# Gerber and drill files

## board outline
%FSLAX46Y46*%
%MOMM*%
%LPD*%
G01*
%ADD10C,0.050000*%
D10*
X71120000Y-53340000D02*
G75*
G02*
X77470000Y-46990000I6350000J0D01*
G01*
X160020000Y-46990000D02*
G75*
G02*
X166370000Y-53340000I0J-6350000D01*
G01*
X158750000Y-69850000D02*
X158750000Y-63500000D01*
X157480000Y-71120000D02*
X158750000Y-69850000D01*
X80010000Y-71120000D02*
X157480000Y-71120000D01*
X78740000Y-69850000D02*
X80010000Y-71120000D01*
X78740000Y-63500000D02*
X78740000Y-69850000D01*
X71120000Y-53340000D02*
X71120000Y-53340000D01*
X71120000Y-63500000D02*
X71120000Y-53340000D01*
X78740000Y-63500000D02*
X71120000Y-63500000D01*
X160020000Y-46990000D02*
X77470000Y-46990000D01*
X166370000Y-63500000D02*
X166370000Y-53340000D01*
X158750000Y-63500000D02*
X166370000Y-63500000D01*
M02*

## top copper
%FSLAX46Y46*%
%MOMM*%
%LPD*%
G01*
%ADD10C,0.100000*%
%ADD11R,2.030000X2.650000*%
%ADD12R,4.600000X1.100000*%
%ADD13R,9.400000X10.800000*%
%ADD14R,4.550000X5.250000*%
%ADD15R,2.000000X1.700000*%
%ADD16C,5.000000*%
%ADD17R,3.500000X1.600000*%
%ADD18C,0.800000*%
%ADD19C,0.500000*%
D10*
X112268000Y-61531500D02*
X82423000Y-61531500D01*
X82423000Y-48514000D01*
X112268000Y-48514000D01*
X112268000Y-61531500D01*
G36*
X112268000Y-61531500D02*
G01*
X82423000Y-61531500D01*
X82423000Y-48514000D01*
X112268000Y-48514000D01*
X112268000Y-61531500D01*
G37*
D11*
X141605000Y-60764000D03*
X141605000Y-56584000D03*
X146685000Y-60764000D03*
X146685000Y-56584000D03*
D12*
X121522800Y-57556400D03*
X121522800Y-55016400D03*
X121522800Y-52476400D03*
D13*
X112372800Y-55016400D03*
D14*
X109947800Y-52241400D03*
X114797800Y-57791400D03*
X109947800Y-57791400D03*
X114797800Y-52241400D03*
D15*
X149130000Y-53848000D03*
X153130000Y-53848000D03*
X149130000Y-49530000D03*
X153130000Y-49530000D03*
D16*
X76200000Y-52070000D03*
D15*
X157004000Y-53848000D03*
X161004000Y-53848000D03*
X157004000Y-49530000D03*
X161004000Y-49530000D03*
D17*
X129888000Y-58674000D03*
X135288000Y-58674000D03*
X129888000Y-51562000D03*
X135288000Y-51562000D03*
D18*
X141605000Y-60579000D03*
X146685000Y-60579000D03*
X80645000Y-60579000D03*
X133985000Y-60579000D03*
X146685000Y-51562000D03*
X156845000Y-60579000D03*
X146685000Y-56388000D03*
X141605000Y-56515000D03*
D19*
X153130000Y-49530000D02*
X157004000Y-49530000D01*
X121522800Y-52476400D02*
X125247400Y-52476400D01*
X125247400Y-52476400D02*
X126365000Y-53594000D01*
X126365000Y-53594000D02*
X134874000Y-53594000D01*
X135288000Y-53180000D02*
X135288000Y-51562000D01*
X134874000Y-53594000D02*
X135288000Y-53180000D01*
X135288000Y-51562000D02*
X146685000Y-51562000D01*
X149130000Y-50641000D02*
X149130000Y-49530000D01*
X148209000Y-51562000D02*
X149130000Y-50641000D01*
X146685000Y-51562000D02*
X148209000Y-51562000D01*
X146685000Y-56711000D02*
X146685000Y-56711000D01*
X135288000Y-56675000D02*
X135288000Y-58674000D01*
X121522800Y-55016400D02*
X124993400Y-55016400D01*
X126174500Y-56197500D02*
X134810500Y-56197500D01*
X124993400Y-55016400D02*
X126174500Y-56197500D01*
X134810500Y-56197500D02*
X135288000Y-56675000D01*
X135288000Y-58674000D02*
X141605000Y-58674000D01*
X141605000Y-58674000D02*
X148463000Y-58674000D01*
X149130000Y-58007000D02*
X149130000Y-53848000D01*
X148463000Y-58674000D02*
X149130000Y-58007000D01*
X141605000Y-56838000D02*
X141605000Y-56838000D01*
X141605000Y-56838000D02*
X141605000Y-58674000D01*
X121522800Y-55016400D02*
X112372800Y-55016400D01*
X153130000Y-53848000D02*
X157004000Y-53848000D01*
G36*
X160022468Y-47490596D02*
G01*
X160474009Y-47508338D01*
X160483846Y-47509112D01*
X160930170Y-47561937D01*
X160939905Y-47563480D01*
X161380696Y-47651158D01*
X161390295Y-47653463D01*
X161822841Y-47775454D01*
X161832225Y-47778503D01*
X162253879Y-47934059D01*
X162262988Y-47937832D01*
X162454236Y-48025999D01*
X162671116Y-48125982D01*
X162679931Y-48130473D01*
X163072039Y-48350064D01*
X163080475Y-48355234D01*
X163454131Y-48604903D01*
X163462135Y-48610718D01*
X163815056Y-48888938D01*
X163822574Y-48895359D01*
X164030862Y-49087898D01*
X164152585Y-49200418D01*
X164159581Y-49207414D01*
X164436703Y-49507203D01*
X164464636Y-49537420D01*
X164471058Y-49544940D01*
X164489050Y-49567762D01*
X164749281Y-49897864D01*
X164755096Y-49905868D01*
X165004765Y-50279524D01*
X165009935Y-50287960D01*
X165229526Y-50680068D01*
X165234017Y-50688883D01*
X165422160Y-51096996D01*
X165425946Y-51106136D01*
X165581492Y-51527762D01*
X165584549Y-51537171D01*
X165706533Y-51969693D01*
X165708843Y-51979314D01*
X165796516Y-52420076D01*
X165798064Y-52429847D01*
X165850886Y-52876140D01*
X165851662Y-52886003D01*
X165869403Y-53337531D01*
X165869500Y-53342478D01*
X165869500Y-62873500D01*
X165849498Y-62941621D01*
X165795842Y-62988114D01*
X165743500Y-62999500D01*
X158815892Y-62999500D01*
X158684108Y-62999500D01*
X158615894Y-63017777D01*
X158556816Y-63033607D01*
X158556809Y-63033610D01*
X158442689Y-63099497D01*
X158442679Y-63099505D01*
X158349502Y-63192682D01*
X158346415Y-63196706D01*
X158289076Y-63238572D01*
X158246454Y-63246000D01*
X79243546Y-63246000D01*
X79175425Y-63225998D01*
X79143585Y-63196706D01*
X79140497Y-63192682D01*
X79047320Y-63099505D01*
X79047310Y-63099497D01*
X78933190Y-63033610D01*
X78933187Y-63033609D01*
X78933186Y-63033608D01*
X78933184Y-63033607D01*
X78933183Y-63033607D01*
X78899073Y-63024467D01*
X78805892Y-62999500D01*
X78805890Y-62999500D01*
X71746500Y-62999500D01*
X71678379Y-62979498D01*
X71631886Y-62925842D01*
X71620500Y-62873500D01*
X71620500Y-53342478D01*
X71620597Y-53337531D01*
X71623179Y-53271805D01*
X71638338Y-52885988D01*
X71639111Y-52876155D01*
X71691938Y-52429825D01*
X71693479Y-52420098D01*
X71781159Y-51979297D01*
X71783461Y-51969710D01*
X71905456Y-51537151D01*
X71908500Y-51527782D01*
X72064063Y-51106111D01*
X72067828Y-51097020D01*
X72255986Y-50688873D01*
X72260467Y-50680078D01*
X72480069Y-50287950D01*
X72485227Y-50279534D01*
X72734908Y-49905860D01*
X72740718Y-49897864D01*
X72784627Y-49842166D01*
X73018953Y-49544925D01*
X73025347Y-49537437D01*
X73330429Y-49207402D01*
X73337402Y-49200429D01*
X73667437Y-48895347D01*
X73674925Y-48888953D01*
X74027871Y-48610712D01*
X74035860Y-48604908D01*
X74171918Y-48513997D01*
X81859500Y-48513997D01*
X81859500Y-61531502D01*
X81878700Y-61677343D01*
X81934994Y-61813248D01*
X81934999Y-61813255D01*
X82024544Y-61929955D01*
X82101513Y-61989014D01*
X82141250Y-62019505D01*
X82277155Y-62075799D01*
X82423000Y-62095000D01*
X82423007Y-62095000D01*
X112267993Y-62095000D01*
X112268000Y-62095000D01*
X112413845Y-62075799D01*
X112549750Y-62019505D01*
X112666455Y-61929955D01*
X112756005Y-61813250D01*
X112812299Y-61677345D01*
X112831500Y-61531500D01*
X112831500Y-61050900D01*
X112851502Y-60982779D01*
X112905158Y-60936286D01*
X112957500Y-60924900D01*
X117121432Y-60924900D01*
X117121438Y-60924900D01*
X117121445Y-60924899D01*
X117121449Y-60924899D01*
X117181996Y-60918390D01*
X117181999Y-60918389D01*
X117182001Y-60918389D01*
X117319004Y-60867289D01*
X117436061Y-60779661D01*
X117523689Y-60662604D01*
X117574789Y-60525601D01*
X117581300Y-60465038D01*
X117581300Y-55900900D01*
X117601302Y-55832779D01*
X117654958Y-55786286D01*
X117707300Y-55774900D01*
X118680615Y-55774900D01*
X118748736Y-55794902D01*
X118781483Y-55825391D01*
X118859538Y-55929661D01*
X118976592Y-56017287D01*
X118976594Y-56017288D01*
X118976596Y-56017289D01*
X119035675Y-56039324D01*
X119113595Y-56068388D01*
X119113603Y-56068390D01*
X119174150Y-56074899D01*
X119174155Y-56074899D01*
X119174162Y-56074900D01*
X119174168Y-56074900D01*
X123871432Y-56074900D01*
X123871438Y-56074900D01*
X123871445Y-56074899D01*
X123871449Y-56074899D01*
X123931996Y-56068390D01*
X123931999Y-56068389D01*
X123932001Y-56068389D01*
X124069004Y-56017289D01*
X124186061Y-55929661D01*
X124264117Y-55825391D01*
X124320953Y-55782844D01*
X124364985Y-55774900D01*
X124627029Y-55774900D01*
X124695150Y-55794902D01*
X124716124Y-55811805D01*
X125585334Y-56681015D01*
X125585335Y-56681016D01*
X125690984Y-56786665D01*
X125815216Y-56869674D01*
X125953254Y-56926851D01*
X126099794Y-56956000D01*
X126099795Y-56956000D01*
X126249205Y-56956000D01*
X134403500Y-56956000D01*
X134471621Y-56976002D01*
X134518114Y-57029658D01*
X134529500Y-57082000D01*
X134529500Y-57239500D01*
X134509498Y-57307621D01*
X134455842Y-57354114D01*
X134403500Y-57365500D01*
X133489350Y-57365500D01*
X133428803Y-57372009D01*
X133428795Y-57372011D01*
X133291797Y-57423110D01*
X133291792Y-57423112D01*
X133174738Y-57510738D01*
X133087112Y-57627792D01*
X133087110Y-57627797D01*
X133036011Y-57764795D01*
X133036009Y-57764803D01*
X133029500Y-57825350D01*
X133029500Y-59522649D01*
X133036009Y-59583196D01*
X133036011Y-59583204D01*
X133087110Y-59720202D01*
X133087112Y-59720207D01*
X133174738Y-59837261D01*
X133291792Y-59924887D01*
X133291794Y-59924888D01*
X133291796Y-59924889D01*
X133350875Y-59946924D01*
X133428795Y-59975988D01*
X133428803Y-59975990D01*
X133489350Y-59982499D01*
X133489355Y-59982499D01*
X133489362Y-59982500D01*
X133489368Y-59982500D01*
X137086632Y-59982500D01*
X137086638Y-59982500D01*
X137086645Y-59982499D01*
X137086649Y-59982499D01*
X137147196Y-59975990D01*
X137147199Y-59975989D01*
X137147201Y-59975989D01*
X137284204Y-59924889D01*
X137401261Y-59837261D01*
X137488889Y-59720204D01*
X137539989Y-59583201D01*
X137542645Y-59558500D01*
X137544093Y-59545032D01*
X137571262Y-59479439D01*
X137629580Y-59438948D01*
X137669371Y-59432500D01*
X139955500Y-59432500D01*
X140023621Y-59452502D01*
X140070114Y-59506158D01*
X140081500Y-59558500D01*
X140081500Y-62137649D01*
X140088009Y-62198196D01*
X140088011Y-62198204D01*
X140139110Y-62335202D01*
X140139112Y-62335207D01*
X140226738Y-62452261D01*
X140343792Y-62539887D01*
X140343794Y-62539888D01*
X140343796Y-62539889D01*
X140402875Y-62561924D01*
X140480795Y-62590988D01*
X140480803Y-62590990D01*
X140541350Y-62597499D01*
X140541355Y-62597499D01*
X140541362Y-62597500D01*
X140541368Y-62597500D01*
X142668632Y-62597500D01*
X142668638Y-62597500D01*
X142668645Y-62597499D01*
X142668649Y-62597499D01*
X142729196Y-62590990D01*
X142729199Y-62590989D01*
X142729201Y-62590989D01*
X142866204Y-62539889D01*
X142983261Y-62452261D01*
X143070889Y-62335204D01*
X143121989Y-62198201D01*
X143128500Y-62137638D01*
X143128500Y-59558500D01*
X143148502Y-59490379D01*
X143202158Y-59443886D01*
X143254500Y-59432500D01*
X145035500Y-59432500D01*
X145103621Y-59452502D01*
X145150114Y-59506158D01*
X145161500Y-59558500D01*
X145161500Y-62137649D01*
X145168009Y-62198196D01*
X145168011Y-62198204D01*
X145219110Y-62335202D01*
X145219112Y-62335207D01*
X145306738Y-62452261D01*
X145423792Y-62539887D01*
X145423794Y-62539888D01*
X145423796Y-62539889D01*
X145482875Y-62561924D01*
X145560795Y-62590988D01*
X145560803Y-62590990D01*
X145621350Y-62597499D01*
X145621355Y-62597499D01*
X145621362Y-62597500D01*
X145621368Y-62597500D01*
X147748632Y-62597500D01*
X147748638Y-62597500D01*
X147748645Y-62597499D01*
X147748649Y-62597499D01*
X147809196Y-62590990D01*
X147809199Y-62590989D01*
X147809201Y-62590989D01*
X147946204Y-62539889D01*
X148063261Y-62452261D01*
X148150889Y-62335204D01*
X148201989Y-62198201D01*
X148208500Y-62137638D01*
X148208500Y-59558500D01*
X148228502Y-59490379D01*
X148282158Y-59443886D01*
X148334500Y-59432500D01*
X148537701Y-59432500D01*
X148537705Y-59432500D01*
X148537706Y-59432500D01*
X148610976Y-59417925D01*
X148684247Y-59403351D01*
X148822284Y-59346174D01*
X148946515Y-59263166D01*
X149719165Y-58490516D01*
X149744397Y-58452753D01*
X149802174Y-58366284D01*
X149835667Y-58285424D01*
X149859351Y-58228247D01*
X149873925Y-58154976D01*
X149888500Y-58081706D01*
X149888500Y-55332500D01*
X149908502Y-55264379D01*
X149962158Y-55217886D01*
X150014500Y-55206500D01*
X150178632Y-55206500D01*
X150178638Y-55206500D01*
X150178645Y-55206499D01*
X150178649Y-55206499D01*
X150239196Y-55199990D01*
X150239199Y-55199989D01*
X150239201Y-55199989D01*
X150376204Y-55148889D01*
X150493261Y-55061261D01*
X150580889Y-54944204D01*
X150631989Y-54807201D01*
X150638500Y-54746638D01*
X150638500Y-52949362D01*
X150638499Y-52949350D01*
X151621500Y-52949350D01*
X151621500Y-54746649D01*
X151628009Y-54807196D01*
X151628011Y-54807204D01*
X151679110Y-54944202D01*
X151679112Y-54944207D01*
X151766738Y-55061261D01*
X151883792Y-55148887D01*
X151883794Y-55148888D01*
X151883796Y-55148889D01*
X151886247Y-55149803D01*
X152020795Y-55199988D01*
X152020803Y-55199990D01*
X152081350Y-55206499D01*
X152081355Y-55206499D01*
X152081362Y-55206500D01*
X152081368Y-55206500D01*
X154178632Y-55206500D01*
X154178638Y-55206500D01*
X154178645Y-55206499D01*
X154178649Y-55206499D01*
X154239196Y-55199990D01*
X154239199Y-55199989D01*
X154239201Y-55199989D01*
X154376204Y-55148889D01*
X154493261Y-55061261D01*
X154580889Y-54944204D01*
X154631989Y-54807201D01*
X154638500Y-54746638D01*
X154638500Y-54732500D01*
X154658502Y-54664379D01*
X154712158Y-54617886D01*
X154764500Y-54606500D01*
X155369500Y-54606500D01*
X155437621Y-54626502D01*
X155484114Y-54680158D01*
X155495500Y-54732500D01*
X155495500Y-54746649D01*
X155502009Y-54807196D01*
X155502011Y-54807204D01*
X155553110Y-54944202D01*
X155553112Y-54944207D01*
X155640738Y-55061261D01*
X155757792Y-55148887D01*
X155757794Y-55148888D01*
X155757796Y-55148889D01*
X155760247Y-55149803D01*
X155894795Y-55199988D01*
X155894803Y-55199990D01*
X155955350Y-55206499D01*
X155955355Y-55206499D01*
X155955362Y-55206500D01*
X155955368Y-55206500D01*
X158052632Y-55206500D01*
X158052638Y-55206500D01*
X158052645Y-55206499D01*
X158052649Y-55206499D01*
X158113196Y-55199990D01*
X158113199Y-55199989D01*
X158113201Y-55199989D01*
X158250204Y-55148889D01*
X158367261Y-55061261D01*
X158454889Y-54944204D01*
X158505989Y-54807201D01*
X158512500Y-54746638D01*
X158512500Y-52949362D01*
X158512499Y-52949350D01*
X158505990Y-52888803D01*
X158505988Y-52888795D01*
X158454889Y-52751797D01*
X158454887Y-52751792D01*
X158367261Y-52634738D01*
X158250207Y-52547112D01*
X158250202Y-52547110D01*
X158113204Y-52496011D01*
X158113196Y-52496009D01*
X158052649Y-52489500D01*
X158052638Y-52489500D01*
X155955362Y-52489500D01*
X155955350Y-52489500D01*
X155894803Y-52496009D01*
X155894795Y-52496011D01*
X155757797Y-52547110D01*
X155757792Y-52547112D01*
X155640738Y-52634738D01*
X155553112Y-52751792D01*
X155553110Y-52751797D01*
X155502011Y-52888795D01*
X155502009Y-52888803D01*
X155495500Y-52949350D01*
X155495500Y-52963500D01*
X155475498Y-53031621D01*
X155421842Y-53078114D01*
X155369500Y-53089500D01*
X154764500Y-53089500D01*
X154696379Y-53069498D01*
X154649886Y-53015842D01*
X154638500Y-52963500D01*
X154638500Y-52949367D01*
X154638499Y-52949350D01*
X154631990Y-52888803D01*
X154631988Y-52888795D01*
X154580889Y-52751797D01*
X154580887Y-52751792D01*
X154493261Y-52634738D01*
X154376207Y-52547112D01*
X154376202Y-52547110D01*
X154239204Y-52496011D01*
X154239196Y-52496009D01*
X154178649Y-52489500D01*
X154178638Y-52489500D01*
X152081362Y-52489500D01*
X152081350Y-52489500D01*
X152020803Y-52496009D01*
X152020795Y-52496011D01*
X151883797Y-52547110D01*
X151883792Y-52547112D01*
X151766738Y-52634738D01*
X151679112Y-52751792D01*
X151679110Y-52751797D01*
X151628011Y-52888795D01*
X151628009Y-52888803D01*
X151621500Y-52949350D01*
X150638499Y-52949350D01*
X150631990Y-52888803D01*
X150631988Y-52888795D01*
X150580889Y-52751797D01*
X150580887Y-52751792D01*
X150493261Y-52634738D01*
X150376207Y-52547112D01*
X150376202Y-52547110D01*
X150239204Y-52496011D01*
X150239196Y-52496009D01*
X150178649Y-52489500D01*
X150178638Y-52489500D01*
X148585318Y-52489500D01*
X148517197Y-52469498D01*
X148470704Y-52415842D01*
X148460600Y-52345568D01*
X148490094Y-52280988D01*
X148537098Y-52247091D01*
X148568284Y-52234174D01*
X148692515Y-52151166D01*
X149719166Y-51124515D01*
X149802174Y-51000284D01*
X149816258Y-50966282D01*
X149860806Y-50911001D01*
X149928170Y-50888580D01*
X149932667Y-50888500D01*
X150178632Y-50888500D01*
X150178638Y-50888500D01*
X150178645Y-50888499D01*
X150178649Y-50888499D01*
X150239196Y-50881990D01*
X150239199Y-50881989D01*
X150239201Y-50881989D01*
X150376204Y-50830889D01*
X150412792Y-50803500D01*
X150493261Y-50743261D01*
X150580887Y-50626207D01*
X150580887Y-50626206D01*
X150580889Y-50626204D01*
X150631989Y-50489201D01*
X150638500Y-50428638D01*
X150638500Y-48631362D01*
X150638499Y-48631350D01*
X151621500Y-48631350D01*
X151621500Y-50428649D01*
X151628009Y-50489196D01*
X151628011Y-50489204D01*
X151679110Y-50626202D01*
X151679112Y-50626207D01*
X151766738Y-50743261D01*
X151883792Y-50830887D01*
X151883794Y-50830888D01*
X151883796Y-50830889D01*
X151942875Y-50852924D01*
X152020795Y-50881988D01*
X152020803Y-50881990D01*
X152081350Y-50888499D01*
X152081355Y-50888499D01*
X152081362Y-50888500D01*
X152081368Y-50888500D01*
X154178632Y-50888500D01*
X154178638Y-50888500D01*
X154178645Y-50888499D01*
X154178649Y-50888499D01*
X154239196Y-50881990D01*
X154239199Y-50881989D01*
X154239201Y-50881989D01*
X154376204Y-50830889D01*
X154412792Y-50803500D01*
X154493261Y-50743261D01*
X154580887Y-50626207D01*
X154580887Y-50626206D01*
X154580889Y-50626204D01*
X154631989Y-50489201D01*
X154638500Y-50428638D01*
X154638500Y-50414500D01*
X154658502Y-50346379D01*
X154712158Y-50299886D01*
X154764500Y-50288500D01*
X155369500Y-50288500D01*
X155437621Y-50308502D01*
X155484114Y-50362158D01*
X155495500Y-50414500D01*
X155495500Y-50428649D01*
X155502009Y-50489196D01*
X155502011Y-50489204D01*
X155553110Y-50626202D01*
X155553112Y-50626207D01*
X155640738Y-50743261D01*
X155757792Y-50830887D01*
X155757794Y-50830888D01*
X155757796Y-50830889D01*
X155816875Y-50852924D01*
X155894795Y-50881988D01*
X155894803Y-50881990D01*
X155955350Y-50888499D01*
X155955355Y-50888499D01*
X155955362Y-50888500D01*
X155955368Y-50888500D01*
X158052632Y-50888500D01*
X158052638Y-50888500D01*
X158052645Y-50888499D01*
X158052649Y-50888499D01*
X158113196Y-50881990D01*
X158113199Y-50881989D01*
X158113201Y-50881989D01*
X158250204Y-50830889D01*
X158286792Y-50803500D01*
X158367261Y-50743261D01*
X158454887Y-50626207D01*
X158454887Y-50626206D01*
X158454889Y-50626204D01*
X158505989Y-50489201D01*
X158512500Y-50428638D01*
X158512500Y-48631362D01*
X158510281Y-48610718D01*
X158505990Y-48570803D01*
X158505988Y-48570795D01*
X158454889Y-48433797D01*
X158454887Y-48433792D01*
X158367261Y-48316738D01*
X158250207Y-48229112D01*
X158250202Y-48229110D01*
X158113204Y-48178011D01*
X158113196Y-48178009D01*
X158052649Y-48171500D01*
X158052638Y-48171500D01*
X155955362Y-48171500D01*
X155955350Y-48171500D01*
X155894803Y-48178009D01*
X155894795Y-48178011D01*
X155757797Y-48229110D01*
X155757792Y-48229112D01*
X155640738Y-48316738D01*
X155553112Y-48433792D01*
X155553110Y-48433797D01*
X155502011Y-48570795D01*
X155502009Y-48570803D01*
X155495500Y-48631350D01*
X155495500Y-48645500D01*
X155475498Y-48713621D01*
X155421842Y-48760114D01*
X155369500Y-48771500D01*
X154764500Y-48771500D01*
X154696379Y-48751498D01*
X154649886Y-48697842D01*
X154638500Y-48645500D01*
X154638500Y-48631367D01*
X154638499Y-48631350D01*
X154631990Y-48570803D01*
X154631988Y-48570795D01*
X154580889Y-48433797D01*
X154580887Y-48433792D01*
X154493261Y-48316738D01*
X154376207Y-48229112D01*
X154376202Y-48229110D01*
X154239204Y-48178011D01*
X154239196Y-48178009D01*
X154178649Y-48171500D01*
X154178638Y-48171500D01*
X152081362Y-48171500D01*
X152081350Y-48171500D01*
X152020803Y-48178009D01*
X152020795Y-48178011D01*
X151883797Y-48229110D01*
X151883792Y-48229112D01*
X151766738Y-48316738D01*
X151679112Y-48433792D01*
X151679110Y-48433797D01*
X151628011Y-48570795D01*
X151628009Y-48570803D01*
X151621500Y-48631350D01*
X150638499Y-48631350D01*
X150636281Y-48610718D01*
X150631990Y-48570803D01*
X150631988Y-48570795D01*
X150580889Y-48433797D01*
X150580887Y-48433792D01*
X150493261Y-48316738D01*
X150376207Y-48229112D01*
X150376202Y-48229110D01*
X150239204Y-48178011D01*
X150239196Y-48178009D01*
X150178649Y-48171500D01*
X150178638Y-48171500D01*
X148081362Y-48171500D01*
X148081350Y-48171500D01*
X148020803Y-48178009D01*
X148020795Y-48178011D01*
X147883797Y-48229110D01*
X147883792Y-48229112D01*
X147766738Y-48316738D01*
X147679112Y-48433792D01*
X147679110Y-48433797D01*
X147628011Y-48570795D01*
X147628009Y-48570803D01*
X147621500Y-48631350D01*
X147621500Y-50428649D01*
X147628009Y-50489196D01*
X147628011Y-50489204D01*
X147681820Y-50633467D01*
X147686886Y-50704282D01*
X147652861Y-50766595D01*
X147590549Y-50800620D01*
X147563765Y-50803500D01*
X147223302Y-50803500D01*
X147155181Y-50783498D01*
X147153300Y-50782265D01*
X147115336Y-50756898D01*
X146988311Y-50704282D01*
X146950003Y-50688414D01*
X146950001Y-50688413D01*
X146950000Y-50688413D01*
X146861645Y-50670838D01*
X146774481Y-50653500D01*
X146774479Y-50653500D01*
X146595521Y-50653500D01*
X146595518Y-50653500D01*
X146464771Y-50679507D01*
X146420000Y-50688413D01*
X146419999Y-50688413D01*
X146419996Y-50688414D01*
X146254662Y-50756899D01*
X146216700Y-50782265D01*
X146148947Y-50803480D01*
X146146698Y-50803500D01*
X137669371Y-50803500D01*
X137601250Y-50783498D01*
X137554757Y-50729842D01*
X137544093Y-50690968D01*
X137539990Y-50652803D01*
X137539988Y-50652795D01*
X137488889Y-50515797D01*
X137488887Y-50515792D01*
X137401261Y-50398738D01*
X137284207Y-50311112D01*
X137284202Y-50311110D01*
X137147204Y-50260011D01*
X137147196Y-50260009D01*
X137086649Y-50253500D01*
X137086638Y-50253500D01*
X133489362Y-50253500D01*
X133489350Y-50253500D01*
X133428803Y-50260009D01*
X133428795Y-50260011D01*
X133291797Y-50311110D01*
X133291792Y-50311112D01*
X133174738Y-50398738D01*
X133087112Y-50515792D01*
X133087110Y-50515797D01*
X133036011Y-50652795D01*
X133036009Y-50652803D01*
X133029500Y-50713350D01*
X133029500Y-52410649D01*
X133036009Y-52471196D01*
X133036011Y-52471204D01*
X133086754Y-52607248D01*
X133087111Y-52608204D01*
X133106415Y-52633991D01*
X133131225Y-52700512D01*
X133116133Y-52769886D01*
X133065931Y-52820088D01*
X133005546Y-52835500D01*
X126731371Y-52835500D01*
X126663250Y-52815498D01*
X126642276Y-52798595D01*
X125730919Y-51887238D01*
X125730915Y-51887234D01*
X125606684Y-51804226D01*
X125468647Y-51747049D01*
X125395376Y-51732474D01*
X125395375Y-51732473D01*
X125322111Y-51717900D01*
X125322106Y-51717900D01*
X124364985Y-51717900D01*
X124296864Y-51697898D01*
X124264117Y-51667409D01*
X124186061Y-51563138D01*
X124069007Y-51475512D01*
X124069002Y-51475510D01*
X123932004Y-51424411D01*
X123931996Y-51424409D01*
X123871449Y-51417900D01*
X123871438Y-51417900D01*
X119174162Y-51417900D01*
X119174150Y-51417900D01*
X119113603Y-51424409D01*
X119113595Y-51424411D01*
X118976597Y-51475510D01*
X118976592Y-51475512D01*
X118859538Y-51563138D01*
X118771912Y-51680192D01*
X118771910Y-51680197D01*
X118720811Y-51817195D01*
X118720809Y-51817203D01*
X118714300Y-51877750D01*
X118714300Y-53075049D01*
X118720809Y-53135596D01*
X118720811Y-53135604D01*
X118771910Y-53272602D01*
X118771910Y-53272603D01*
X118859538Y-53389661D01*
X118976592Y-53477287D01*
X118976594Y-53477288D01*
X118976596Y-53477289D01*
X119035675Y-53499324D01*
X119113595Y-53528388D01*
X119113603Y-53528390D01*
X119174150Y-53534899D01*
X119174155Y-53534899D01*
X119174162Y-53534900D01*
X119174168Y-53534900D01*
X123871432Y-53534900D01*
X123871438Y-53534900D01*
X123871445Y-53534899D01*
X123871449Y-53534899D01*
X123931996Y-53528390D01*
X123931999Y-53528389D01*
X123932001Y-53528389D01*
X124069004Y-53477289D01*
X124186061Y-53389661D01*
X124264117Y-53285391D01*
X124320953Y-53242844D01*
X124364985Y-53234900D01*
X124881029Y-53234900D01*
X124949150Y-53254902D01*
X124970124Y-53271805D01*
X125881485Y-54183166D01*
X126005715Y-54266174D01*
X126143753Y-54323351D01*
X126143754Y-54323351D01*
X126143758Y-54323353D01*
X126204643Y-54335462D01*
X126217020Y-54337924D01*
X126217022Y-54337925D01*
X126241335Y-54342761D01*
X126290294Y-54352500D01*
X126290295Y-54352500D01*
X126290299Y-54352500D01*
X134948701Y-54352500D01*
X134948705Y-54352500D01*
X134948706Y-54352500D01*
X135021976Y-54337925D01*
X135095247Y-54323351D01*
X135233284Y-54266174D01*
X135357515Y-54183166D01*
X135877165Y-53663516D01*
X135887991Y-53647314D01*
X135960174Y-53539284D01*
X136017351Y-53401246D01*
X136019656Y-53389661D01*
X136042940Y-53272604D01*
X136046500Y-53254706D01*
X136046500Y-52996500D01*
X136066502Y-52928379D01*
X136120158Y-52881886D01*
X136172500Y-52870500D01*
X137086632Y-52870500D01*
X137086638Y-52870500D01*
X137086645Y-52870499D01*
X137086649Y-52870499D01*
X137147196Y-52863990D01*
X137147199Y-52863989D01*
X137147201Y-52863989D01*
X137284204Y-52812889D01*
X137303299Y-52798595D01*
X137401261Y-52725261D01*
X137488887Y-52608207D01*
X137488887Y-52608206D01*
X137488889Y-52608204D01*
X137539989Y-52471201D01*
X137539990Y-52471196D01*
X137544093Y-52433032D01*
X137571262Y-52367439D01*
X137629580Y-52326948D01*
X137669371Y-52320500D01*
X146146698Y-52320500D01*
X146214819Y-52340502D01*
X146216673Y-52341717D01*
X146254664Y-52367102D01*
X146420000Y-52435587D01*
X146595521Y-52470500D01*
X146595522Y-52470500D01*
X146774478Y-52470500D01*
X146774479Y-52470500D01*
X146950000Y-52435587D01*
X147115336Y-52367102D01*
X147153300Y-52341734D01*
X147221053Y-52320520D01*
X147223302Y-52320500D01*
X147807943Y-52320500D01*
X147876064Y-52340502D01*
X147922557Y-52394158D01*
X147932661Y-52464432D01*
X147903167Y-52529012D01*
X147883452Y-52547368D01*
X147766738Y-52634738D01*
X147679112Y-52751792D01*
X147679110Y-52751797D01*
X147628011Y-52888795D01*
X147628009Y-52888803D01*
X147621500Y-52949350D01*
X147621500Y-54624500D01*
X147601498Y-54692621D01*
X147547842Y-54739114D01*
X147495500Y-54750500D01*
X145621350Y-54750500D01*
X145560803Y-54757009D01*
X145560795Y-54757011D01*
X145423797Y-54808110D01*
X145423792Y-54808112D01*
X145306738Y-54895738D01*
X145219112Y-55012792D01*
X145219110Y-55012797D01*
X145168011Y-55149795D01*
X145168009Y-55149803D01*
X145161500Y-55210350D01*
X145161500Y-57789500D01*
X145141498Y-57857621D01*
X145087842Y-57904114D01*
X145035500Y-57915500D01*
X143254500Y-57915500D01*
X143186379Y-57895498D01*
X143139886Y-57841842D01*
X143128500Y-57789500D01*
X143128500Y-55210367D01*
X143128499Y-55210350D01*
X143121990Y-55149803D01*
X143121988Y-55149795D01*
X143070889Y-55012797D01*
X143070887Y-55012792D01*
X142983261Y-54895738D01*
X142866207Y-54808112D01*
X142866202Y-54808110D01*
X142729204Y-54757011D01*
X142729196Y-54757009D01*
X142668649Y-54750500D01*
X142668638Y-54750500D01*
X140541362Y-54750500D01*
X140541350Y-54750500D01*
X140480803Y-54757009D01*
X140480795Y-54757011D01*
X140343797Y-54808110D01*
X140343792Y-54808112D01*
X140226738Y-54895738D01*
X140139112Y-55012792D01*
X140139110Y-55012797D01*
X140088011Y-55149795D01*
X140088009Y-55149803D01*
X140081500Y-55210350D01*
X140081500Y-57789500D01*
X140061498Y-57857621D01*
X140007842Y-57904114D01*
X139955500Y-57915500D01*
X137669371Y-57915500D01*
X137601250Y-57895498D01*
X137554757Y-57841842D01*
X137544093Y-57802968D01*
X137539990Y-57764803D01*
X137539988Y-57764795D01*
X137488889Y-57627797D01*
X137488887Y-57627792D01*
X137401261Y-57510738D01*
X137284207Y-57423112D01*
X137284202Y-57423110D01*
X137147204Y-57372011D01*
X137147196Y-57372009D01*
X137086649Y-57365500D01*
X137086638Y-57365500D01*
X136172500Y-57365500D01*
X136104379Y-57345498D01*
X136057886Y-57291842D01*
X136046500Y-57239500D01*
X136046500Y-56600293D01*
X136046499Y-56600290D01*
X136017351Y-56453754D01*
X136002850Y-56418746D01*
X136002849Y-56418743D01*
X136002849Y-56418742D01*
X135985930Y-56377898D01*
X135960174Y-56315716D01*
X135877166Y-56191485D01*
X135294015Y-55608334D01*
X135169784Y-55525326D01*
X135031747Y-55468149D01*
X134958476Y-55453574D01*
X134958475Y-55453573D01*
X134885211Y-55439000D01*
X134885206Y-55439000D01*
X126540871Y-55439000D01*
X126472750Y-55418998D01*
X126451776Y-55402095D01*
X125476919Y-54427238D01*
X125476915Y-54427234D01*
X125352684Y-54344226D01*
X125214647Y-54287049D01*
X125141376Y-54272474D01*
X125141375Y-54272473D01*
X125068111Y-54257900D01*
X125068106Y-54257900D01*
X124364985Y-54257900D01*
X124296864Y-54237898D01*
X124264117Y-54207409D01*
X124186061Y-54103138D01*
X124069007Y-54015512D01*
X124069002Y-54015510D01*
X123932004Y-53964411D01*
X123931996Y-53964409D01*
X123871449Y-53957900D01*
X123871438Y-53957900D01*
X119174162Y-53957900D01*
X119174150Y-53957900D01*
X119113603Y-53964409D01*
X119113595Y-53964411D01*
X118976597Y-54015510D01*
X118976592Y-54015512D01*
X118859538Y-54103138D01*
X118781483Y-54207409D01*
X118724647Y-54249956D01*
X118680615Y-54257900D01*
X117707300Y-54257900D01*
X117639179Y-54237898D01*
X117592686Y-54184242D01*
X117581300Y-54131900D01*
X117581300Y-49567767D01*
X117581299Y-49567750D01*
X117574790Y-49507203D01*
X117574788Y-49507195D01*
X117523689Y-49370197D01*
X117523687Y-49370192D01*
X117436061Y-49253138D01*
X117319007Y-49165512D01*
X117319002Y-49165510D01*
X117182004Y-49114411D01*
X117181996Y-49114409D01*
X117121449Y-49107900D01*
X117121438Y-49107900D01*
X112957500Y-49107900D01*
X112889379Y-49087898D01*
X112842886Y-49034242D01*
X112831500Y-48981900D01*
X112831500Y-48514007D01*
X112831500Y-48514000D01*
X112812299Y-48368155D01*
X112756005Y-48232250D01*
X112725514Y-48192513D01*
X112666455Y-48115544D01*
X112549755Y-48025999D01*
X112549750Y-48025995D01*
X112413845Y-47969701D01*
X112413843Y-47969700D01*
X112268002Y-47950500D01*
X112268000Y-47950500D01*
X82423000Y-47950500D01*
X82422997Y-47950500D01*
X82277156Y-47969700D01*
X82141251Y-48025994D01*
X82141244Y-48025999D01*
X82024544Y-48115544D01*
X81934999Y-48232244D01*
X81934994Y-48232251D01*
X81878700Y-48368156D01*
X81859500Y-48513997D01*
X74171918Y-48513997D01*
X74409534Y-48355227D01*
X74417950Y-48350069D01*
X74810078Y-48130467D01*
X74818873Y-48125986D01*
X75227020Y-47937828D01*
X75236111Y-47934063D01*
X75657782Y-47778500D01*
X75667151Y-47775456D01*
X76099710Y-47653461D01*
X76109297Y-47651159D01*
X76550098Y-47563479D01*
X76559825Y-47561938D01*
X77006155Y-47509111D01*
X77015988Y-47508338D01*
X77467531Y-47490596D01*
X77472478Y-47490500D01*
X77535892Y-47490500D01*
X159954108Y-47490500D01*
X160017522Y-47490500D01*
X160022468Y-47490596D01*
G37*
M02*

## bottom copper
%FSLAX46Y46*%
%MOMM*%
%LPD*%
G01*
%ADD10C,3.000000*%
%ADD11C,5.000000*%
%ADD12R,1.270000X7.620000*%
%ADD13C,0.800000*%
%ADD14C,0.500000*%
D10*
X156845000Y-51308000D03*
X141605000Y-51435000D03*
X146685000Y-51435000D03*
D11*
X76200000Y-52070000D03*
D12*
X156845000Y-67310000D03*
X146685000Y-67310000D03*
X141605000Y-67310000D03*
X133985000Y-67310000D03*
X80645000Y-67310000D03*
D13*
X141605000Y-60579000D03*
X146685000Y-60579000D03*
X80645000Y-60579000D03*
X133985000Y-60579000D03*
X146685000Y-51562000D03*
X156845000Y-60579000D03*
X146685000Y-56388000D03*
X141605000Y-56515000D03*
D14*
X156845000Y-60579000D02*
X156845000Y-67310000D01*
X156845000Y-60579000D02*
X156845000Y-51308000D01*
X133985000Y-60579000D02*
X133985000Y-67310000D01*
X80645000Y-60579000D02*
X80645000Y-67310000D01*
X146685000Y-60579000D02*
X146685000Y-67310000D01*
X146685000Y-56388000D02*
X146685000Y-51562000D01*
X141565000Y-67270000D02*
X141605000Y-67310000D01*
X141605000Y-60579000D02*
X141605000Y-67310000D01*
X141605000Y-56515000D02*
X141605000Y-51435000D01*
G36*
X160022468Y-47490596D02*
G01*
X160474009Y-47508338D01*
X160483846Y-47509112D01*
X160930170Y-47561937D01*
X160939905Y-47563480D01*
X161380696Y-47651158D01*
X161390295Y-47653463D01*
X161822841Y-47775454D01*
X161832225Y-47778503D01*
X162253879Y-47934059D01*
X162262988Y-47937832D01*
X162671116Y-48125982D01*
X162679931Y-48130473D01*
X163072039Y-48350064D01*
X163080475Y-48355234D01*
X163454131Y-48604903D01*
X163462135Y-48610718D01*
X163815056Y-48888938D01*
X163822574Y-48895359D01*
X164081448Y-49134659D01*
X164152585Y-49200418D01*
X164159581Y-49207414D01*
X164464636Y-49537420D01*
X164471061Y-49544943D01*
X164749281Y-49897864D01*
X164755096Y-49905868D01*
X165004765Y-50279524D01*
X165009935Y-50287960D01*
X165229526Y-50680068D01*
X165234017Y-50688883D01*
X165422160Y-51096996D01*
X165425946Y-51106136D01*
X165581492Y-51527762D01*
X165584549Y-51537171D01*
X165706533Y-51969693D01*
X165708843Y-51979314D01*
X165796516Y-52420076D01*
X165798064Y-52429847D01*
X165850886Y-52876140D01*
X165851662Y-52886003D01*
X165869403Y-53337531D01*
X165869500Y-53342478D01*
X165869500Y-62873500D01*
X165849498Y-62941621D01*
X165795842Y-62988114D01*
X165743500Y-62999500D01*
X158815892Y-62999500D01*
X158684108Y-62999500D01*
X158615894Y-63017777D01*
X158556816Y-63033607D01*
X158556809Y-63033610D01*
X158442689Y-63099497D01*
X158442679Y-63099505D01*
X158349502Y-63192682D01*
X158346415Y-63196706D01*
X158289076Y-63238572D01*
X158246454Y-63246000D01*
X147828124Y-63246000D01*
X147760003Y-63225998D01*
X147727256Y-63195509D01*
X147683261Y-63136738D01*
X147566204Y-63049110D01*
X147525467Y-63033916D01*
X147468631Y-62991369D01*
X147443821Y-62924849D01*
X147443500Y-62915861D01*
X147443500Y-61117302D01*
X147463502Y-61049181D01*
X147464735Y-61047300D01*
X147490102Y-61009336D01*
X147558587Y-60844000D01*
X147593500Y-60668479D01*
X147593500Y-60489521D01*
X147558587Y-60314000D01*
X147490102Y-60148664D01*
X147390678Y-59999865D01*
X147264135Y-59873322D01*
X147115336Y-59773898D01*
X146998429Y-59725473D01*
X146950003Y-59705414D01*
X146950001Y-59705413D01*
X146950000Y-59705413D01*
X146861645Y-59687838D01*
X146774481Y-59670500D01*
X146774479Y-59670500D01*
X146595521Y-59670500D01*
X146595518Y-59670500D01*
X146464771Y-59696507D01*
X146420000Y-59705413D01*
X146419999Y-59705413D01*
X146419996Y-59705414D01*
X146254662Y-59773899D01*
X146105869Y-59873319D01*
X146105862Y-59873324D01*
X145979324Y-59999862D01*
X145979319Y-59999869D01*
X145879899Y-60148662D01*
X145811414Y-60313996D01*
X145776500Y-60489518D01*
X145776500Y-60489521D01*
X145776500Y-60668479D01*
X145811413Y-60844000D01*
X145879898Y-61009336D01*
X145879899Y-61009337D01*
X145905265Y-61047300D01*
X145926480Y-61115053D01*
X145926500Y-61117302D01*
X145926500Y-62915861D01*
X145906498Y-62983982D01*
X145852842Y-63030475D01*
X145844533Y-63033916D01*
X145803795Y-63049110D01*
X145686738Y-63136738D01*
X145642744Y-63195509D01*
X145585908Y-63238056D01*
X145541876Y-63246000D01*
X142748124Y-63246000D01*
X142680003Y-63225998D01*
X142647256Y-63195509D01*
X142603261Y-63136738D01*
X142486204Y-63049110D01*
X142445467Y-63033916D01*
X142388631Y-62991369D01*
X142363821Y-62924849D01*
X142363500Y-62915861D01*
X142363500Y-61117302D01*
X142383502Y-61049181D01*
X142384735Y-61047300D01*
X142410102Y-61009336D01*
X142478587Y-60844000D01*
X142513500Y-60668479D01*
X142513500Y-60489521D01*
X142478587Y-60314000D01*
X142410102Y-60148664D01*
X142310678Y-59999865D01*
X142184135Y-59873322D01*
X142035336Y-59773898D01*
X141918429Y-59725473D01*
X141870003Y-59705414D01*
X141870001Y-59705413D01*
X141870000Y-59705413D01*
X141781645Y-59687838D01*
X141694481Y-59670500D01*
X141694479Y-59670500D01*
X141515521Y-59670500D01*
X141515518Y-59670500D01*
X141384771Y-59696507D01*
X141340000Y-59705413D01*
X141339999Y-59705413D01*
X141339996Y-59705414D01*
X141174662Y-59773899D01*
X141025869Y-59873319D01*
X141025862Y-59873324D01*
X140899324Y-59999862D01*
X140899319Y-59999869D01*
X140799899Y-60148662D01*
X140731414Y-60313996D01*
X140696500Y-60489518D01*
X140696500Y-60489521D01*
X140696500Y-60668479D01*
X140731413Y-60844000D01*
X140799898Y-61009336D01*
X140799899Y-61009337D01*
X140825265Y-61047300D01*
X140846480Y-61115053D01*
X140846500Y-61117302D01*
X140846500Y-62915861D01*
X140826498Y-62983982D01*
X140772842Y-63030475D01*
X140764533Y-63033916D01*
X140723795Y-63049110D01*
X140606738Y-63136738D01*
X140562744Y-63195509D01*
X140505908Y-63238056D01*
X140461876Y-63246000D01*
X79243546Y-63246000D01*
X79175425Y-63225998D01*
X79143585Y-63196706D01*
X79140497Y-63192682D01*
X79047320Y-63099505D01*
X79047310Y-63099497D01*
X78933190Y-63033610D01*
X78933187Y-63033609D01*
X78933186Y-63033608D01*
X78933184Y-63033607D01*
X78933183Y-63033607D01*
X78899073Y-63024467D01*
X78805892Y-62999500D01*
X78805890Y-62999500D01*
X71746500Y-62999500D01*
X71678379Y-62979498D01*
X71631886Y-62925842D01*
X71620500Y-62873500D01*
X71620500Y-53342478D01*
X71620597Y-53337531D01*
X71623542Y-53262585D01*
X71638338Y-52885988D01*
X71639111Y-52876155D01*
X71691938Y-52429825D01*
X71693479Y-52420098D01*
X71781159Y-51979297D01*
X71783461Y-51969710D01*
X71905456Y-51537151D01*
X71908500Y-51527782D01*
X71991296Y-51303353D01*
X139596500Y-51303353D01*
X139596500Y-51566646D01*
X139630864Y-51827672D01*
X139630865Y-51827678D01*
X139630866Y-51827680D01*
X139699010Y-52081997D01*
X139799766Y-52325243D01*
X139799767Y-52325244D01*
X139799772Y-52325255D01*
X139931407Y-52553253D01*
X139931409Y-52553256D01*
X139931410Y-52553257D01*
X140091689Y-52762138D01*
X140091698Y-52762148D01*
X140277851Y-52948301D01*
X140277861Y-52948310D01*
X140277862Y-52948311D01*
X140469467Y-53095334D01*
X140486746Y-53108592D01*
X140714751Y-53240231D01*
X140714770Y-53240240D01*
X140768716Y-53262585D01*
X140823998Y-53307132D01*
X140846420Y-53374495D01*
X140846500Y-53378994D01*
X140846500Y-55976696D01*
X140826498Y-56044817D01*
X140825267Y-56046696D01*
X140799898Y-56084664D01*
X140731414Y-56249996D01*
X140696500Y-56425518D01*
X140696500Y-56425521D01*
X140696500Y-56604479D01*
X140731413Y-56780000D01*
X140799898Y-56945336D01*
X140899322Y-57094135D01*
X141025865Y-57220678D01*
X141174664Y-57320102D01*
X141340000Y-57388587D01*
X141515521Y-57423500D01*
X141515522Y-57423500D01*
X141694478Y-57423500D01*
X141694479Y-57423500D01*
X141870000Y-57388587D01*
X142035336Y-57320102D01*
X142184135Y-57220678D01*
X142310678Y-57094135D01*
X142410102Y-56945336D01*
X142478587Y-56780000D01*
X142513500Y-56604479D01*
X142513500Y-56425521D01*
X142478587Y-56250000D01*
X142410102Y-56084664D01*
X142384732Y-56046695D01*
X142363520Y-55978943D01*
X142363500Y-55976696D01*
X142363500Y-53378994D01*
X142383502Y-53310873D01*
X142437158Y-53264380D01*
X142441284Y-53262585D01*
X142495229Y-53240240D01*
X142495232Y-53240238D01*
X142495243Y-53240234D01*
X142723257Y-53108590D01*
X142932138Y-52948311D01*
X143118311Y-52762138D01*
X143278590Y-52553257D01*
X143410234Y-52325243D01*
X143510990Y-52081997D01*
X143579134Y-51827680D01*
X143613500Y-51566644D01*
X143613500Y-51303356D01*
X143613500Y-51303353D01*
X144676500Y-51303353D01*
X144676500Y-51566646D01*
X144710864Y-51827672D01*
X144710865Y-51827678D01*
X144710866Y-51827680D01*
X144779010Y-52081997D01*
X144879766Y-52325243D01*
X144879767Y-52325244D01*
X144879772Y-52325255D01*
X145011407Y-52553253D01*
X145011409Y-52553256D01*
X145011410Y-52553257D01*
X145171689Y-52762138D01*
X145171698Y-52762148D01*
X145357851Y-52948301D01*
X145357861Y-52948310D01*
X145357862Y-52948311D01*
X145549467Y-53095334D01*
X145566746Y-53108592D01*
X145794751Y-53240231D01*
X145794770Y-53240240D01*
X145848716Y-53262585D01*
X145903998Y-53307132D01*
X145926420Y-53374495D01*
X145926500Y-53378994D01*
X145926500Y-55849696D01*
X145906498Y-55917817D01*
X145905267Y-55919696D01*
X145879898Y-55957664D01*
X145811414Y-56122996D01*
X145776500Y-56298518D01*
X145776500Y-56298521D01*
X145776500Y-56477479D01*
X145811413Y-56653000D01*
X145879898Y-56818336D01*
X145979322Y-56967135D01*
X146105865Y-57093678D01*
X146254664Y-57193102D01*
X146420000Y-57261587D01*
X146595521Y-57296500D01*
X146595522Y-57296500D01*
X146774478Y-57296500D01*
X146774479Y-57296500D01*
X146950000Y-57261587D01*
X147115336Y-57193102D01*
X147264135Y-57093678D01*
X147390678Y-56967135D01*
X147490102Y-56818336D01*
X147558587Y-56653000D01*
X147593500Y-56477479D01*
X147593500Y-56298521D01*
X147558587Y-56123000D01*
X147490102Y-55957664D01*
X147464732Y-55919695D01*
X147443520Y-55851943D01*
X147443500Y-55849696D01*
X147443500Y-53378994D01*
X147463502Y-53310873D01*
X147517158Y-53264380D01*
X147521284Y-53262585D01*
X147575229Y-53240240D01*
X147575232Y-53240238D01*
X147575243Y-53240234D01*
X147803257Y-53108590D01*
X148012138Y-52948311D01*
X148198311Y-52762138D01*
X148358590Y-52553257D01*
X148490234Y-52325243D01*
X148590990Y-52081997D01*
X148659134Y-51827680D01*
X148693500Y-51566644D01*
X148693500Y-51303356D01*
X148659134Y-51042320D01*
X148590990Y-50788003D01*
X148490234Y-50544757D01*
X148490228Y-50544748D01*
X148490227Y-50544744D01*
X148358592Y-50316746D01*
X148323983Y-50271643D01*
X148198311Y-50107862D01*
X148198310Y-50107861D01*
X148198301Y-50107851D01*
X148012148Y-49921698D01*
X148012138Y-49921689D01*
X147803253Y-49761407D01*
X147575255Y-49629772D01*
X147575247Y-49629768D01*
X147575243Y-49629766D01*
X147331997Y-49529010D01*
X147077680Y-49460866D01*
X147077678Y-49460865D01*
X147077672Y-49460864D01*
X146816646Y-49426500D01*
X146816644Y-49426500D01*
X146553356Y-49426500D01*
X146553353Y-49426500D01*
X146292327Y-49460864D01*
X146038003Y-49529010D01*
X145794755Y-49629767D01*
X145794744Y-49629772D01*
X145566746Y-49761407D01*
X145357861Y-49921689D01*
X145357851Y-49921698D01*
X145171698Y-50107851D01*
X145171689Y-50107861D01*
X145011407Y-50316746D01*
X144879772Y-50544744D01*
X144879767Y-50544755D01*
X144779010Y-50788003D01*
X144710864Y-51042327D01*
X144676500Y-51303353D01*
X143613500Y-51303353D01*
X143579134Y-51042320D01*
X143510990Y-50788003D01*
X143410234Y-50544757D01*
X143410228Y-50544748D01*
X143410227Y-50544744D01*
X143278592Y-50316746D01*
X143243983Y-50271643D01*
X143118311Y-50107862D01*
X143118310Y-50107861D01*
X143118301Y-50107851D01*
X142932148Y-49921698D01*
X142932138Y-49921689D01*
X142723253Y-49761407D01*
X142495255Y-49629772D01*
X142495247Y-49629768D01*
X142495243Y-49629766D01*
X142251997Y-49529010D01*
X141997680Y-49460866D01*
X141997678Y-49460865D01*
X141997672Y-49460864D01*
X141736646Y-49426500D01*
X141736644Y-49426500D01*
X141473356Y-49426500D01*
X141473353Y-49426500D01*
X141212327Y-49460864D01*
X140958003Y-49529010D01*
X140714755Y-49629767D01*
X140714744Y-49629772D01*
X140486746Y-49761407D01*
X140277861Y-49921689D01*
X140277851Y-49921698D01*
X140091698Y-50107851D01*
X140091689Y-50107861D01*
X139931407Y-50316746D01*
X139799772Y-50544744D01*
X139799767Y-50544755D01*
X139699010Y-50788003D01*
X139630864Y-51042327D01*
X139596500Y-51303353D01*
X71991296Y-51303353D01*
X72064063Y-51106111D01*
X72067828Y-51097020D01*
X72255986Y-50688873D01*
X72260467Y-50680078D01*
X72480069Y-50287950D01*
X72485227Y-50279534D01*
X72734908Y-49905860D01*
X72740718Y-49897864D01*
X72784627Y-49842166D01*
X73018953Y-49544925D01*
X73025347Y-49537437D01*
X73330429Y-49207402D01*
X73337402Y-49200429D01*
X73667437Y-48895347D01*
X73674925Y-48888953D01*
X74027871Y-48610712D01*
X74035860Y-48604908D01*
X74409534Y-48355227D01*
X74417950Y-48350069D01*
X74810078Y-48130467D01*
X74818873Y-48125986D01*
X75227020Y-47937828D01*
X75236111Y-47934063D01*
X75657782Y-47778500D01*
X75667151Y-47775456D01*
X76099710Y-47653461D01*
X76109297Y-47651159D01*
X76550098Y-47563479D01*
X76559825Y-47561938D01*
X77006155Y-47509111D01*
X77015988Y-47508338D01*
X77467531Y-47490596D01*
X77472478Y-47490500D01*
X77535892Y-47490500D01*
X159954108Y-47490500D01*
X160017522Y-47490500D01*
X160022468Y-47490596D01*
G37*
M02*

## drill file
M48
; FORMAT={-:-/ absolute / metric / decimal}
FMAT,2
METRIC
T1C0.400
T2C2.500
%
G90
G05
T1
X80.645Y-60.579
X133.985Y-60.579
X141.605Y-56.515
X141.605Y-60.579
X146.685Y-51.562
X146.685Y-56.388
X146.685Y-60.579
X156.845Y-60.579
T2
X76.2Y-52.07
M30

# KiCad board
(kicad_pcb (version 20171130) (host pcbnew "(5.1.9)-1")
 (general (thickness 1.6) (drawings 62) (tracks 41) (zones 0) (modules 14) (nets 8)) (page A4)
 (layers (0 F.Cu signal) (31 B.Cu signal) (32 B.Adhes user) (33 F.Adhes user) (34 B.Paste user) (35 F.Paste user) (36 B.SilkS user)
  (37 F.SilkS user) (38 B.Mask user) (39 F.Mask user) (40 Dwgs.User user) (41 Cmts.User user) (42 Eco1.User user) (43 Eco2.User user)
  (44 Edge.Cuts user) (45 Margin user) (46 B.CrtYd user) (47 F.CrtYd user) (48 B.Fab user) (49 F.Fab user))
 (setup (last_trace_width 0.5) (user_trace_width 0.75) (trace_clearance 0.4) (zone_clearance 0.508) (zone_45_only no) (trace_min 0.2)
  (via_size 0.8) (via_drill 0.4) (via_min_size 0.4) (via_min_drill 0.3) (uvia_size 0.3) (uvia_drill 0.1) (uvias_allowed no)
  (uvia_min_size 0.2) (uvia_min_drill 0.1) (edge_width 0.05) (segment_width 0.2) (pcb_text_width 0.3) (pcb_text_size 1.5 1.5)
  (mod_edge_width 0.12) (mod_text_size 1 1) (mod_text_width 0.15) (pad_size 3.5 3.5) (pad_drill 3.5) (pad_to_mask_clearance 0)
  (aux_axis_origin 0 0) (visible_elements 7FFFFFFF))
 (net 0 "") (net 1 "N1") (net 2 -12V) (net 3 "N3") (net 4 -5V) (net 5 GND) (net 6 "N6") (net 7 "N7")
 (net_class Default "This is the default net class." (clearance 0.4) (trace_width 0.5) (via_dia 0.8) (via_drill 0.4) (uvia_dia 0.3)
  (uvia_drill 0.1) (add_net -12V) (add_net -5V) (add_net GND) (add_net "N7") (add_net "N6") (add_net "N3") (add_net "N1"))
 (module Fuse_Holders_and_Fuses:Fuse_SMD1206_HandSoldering (layer F.Cu) (at 141.605 58.674 90)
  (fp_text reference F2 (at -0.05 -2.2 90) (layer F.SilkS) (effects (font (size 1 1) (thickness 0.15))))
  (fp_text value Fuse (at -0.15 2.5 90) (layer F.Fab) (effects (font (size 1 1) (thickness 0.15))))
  (pad 1 smd rect (at -2.09 0 180) (size 2.03 2.65) (layers F.Cu F.Paste F.Mask) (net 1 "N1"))
  (pad 2 smd rect (at 2.09 0 180) (size 2.03 2.65) (layers F.Cu F.Paste F.Mask) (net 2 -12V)))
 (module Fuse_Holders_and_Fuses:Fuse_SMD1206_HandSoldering (layer F.Cu) (at 146.685 58.674 90)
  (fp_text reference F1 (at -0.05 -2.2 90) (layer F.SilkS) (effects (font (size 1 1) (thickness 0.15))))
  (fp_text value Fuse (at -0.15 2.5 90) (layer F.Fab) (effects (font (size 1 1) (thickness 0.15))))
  (pad 1 smd rect (at -2.09 0 180) (size 2.03 2.65) (layers F.Cu F.Paste F.Mask) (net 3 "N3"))
  (pad 2 smd rect (at 2.09 0 180) (size 2.03 2.65) (layers F.Cu F.Paste F.Mask) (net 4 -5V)))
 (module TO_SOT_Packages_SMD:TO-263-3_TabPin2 (layer F.Cu) (at 115.7478 55.0164 180)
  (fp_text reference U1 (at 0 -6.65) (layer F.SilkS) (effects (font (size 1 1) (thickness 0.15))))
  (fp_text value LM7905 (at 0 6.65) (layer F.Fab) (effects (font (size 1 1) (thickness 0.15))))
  (pad 1 smd rect (at -5.775 -2.54 180) (size 4.6 1.1) (layers F.Cu F.Paste F.Mask) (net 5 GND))
  (pad 2 smd rect (at -5.775 0 180) (size 4.6 1.1) (layers F.Cu F.Paste F.Mask) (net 2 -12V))
  (pad 3 smd rect (at -5.775 2.54 180) (size 4.6 1.1) (layers F.Cu F.Paste F.Mask) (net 4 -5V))
  (pad 2 smd rect (at 3.375 0 180) (size 9.4 10.8) (layers F.Cu F.Mask) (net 2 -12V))
  (pad 2 smd rect (at 5.8 2.775 180) (size 4.55 5.25) (layers F.Cu F.Paste) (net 2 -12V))
  (pad 2 smd rect (at 0.95 -2.775 180) (size 4.55 5.25) (layers F.Cu F.Paste) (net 2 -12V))
  (pad 2 smd rect (at 5.8 -2.775 180) (size 4.55 5.25) (layers F.Cu F.Paste) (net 2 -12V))
  (pad 2 smd rect (at 0.95 2.775 180) (size 4.55 5.25) (layers F.Cu F.Paste) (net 2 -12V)))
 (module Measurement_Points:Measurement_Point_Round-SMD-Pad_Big (layer B.Cu) (at 156.845 51.308)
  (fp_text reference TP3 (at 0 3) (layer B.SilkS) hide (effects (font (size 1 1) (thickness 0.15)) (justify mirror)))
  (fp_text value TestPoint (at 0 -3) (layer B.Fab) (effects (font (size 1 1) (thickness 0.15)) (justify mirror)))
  (pad 1 smd circle (at 0 0) (size 3 3) (layers B.Cu B.Mask) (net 5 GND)))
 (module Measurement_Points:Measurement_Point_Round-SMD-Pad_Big (layer B.Cu) (at 141.605 51.435)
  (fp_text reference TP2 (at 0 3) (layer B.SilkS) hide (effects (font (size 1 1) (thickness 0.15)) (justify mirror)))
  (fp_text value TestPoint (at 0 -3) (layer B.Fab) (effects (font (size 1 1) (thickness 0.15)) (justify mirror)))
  (pad 1 smd circle (at 0 0) (size 3 3) (layers B.Cu B.Mask) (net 2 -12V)))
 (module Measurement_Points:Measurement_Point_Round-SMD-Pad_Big (layer B.Cu) (at 146.685 51.435)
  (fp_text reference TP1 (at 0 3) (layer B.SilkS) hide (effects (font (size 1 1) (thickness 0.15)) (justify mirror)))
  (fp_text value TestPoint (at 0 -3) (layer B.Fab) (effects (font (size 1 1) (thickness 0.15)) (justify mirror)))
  (pad 1 smd circle (at 0 0) (size 3 3) (layers B.Cu B.Mask) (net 4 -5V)))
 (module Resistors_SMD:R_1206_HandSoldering (layer F.Cu) (at 151.13 53.848)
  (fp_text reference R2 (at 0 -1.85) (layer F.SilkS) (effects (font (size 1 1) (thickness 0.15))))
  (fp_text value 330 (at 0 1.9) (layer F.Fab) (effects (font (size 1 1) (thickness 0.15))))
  (pad 1 smd rect (at -2 0) (size 2 1.7) (layers F.Cu F.Paste F.Mask) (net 2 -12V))
  (pad 2 smd rect (at 2 0) (size 2 1.7) (layers F.Cu F.Paste F.Mask) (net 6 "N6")))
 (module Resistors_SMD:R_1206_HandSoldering (layer F.Cu) (at 151.13 49.53)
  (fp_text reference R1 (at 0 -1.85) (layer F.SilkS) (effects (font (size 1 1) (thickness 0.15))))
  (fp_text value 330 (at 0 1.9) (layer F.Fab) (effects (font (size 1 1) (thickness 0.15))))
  (pad 1 smd rect (at -2 0) (size 2 1.7) (layers F.Cu F.Paste F.Mask) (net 4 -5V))
  (pad 2 smd rect (at 2 0) (size 2 1.7) (layers F.Cu F.Paste F.Mask) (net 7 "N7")))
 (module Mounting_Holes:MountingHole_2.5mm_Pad (layer F.Cu) (at 76.2 52.07)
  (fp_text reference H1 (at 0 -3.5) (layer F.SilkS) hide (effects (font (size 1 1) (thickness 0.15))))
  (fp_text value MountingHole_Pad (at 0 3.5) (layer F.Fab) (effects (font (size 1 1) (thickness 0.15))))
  (pad 1 thru_hole circle (at 0 0) (size 5 5) (drill 2.5) (layers *.Cu *.Mask) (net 5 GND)))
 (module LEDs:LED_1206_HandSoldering (layer F.Cu) (at 159.004 53.848)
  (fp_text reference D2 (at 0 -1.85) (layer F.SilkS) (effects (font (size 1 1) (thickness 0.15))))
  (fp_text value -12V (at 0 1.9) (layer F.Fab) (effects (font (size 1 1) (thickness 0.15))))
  (pad 1 smd rect (at -2 0) (size 2 1.7) (layers F.Cu F.Paste F.Mask) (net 6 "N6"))
  (pad 2 smd rect (at 2 0) (size 2 1.7) (layers F.Cu F.Paste F.Mask) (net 5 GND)))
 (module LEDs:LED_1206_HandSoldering (layer F.Cu) (at 159.004 49.53)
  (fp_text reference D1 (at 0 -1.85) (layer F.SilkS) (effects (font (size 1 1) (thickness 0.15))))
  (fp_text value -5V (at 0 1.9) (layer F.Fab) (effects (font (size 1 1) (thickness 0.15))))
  (pad 1 smd rect (at -2 0) (size 2 1.7) (layers F.Cu F.Paste F.Mask) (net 7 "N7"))
  (pad 2 smd rect (at 2 0) (size 2 1.7) (layers F.Cu F.Paste F.Mask) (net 5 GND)))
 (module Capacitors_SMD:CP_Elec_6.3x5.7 (layer F.Cu) (at 132.588 58.674)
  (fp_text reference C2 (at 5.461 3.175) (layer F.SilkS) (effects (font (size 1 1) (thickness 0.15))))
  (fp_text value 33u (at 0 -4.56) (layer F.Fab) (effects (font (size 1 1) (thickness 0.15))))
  (pad 1 smd rect (at -2.7 0 180) (size 3.5 1.6) (layers F.Cu F.Paste F.Mask) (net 5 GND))
  (pad 2 smd rect (at 2.7 0 180) (size 3.5 1.6) (layers F.Cu F.Paste F.Mask) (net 2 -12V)))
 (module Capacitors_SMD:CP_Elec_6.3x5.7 (layer F.Cu) (at 132.588 51.562)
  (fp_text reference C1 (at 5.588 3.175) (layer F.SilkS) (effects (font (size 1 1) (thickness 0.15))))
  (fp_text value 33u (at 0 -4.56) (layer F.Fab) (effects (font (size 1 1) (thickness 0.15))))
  (pad 1 smd rect (at -2.7 0 180) (size 3.5 1.6) (layers F.Cu F.Paste F.Mask) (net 5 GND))
  (pad 2 smd rect (at 2.7 0 180) (size 3.5 1.6) (layers F.Cu F.Paste F.Mask) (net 4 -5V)))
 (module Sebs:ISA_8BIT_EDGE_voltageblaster (layer F.Cu) (at 156.845 63.5)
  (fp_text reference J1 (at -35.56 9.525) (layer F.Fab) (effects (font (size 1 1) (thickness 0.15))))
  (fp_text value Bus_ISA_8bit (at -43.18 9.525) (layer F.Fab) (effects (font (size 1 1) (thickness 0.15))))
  (pad 1 connect rect (at 0 3.81) (size 1.27 7.62) (layers B.Cu B.Mask) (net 5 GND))
  (pad 5 connect rect (at -10.16 3.81) (size 1.27 7.62) (layers B.Cu B.Mask) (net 4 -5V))
  (pad 7 connect rect (at -15.24 3.81) (size 1.27 7.62) (layers B.Cu B.Mask) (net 2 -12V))
  (pad 10 connect rect (at -22.86 3.81) (size 1.27 7.62) (layers B.Cu B.Mask) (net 5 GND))
  (pad 31 connect rect (at -76.2 3.81) (size 1.27 7.62) (layers B.Cu B.Mask) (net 5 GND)))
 (gr_poly (pts (xy 112.268 61.5315) (xy 82.423 61.5315) (xy 82.423 48.514) (xy 112.268 48.514)) (layer F.Cu) (width 0.1))
 (gr_arc (start 77.47 53.34) (end 77.47 46.99) (angle -90) (layer Edge.Cuts) (width 0.05))
 (gr_arc (start 160.02 53.34) (end 166.37 53.34) (angle -90) (layer Edge.Cuts) (width 0.05))
 (gr_line (start 158.75 69.85) (end 158.75 63.5) (layer Edge.Cuts) (width 0.05))
 (gr_line (start 157.48 71.12) (end 158.75 69.85) (layer Edge.Cuts) (width 0.05))
 (gr_line (start 80.01 71.12) (end 157.48 71.12) (layer Edge.Cuts) (width 0.05))
 (gr_line (start 78.74 69.85) (end 80.01 71.12) (layer Edge.Cuts) (width 0.05))
 (gr_line (start 78.74 63.5) (end 78.74 69.85) (layer Edge.Cuts) (width 0.05))
 (gr_line (start 71.12 53.34) (end 71.12 53.34) (layer Edge.Cuts) (width 0.05))
 (gr_line (start 71.12 63.5) (end 71.12 53.34) (layer Edge.Cuts) (width 0.05))
 (gr_line (start 78.74 63.5) (end 71.12 63.5) (layer Edge.Cuts) (width 0.05))
 (gr_line (start 160.02 46.99) (end 77.47 46.99) (layer Edge.Cuts) (width 0.05))
 (gr_line (start 166.37 63.5) (end 166.37 53.34) (layer Edge.Cuts) (width 0.05))
 (gr_line (start 158.75 63.5) (end 166.37 63.5) (layer Edge.Cuts) (width 0.05))
 (via (at 141.605 60.579) (size 0.8) (drill 0.4) (layers F.Cu B.Cu) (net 2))
 (via (at 146.685 60.579) (size 0.8) (drill 0.4) (layers F.Cu B.Cu) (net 4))
 (via (at 80.645 60.579) (size 0.8) (drill 0.4) (layers F.Cu B.Cu) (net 5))
 (via (at 133.985 60.579) (size 0.8) (drill 0.4) (layers F.Cu B.Cu) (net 5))
 (via (at 146.685 51.562) (size 0.8) (drill 0.4) (layers F.Cu B.Cu) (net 4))
 (via (at 156.845 60.579) (size 0.8) (drill 0.4) (layers F.Cu B.Cu) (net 5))
 (segment (start 156.845 60.579) (end 156.845 67.31) (width 0.5) (layer B.Cu) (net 5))
 (segment (start 156.845 60.579) (end 156.845 51.308) (width 0.5) (layer B.Cu) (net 5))
 (segment (start 133.985 60.579) (end 133.985 67.31) (width 0.5) (layer B.Cu) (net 5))
 (segment (start 80.645 60.579) (end 80.645 67.31) (width 0.5) (layer B.Cu) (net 5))
 (segment (start 153.13 49.53) (end 157.004 49.53) (width 0.5) (layer F.Cu) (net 7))
 (segment (start 121.5228 52.4764) (end 125.2474 52.4764) (width 0.5) (layer F.Cu) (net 4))
 (segment (start 125.2474 52.4764) (end 126.365 53.594) (width 0.5) (layer F.Cu) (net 4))
 (segment (start 126.365 53.594) (end 134.874 53.594) (width 0.5) (layer F.Cu) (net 4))
 (segment (start 135.288 53.18) (end 135.288 51.562) (width 0.5) (layer F.Cu) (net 4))
 (segment (start 134.874 53.594) (end 135.288 53.18) (width 0.5) (layer F.Cu) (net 4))
 (segment (start 135.288 51.562) (end 146.685 51.562) (width 0.5) (layer F.Cu) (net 4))
 (segment (start 149.13 50.641) (end 149.13 49.53) (width 0.5) (layer F.Cu) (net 4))
 (segment (start 148.209 51.562) (end 149.13 50.641) (width 0.5) (layer F.Cu) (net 4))
 (segment (start 146.685 51.562) (end 148.209 51.562) (width 0.5) (layer F.Cu) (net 4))
 (segment (start 146.685 56.711) (end 146.685 56.711) (width 0.5) (layer F.Cu) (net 4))
 (via (at 146.685 56.388) (size 0.8) (drill 0.4) (layers F.Cu B.Cu) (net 4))
 (segment (start 146.685 60.579) (end 146.685 67.31) (width 0.5) (layer B.Cu) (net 4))
 (segment (start 146.685 56.388) (end 146.685 51.562) (width 0.5) (layer B.Cu) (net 4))
 (segment (start 141.565 67.27) (end 141.605 67.31) (width 0.5) (layer B.Cu) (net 2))
 (segment (start 135.288 56.675) (end 135.288 58.674) (width 0.5) (layer F.Cu) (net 2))
 (segment (start 121.5228 55.0164) (end 124.9934 55.0164) (width 0.5) (layer F.Cu) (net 2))
 (segment (start 126.1745 56.1975) (end 134.8105 56.1975) (width 0.5) (layer F.Cu) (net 2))
 (segment (start 124.9934 55.0164) (end 126.1745 56.1975) (width 0.5) (layer F.Cu) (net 2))
 (segment (start 134.8105 56.1975) (end 135.288 56.675) (width 0.5) (layer F.Cu) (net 2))
 (segment (start 135.288 58.674) (end 141.605 58.674) (width 0.5) (layer F.Cu) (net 2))
 (segment (start 141.605 58.674) (end 148.463 58.674) (width 0.5) (layer F.Cu) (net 2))
 (segment (start 149.13 58.007) (end 149.13 53.848) (width 0.5) (layer F.Cu) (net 2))
 (segment (start 148.463 58.674) (end 149.13 58.007) (width 0.5) (layer F.Cu) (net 2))
 (segment (start 141.605 56.838) (end 141.605 56.838) (width 0.5) (layer F.Cu) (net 2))
 (segment (start 141.605 56.838) (end 141.605 58.674) (width 0.5) (layer F.Cu) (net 2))
 (via (at 141.605 56.515) (size 0.8) (drill 0.4) (layers F.Cu B.Cu) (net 2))
 (segment (start 141.605 60.579) (end 141.605 67.31) (width 0.5) (layer B.Cu) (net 2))
 (segment (start 141.605 56.515) (end 141.605 51.435) (width 0.5) (layer B.Cu) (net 2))
 (segment (start 121.5228 55.0164) (end 112.3728 55.0164) (width 0.5) (layer F.Cu) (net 2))
 (segment (start 153.13 53.848) (end 157.004 53.848) (width 0.5) (layer F.Cu) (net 6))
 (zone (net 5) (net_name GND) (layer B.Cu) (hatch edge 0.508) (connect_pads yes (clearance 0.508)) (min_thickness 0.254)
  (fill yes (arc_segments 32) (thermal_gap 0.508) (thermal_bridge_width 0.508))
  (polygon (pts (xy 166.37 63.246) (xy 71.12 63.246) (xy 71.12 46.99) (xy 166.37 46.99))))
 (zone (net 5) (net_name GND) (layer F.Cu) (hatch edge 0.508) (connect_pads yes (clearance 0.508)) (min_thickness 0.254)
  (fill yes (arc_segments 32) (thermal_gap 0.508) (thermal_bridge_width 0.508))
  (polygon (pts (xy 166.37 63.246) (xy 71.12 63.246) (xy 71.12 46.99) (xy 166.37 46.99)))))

